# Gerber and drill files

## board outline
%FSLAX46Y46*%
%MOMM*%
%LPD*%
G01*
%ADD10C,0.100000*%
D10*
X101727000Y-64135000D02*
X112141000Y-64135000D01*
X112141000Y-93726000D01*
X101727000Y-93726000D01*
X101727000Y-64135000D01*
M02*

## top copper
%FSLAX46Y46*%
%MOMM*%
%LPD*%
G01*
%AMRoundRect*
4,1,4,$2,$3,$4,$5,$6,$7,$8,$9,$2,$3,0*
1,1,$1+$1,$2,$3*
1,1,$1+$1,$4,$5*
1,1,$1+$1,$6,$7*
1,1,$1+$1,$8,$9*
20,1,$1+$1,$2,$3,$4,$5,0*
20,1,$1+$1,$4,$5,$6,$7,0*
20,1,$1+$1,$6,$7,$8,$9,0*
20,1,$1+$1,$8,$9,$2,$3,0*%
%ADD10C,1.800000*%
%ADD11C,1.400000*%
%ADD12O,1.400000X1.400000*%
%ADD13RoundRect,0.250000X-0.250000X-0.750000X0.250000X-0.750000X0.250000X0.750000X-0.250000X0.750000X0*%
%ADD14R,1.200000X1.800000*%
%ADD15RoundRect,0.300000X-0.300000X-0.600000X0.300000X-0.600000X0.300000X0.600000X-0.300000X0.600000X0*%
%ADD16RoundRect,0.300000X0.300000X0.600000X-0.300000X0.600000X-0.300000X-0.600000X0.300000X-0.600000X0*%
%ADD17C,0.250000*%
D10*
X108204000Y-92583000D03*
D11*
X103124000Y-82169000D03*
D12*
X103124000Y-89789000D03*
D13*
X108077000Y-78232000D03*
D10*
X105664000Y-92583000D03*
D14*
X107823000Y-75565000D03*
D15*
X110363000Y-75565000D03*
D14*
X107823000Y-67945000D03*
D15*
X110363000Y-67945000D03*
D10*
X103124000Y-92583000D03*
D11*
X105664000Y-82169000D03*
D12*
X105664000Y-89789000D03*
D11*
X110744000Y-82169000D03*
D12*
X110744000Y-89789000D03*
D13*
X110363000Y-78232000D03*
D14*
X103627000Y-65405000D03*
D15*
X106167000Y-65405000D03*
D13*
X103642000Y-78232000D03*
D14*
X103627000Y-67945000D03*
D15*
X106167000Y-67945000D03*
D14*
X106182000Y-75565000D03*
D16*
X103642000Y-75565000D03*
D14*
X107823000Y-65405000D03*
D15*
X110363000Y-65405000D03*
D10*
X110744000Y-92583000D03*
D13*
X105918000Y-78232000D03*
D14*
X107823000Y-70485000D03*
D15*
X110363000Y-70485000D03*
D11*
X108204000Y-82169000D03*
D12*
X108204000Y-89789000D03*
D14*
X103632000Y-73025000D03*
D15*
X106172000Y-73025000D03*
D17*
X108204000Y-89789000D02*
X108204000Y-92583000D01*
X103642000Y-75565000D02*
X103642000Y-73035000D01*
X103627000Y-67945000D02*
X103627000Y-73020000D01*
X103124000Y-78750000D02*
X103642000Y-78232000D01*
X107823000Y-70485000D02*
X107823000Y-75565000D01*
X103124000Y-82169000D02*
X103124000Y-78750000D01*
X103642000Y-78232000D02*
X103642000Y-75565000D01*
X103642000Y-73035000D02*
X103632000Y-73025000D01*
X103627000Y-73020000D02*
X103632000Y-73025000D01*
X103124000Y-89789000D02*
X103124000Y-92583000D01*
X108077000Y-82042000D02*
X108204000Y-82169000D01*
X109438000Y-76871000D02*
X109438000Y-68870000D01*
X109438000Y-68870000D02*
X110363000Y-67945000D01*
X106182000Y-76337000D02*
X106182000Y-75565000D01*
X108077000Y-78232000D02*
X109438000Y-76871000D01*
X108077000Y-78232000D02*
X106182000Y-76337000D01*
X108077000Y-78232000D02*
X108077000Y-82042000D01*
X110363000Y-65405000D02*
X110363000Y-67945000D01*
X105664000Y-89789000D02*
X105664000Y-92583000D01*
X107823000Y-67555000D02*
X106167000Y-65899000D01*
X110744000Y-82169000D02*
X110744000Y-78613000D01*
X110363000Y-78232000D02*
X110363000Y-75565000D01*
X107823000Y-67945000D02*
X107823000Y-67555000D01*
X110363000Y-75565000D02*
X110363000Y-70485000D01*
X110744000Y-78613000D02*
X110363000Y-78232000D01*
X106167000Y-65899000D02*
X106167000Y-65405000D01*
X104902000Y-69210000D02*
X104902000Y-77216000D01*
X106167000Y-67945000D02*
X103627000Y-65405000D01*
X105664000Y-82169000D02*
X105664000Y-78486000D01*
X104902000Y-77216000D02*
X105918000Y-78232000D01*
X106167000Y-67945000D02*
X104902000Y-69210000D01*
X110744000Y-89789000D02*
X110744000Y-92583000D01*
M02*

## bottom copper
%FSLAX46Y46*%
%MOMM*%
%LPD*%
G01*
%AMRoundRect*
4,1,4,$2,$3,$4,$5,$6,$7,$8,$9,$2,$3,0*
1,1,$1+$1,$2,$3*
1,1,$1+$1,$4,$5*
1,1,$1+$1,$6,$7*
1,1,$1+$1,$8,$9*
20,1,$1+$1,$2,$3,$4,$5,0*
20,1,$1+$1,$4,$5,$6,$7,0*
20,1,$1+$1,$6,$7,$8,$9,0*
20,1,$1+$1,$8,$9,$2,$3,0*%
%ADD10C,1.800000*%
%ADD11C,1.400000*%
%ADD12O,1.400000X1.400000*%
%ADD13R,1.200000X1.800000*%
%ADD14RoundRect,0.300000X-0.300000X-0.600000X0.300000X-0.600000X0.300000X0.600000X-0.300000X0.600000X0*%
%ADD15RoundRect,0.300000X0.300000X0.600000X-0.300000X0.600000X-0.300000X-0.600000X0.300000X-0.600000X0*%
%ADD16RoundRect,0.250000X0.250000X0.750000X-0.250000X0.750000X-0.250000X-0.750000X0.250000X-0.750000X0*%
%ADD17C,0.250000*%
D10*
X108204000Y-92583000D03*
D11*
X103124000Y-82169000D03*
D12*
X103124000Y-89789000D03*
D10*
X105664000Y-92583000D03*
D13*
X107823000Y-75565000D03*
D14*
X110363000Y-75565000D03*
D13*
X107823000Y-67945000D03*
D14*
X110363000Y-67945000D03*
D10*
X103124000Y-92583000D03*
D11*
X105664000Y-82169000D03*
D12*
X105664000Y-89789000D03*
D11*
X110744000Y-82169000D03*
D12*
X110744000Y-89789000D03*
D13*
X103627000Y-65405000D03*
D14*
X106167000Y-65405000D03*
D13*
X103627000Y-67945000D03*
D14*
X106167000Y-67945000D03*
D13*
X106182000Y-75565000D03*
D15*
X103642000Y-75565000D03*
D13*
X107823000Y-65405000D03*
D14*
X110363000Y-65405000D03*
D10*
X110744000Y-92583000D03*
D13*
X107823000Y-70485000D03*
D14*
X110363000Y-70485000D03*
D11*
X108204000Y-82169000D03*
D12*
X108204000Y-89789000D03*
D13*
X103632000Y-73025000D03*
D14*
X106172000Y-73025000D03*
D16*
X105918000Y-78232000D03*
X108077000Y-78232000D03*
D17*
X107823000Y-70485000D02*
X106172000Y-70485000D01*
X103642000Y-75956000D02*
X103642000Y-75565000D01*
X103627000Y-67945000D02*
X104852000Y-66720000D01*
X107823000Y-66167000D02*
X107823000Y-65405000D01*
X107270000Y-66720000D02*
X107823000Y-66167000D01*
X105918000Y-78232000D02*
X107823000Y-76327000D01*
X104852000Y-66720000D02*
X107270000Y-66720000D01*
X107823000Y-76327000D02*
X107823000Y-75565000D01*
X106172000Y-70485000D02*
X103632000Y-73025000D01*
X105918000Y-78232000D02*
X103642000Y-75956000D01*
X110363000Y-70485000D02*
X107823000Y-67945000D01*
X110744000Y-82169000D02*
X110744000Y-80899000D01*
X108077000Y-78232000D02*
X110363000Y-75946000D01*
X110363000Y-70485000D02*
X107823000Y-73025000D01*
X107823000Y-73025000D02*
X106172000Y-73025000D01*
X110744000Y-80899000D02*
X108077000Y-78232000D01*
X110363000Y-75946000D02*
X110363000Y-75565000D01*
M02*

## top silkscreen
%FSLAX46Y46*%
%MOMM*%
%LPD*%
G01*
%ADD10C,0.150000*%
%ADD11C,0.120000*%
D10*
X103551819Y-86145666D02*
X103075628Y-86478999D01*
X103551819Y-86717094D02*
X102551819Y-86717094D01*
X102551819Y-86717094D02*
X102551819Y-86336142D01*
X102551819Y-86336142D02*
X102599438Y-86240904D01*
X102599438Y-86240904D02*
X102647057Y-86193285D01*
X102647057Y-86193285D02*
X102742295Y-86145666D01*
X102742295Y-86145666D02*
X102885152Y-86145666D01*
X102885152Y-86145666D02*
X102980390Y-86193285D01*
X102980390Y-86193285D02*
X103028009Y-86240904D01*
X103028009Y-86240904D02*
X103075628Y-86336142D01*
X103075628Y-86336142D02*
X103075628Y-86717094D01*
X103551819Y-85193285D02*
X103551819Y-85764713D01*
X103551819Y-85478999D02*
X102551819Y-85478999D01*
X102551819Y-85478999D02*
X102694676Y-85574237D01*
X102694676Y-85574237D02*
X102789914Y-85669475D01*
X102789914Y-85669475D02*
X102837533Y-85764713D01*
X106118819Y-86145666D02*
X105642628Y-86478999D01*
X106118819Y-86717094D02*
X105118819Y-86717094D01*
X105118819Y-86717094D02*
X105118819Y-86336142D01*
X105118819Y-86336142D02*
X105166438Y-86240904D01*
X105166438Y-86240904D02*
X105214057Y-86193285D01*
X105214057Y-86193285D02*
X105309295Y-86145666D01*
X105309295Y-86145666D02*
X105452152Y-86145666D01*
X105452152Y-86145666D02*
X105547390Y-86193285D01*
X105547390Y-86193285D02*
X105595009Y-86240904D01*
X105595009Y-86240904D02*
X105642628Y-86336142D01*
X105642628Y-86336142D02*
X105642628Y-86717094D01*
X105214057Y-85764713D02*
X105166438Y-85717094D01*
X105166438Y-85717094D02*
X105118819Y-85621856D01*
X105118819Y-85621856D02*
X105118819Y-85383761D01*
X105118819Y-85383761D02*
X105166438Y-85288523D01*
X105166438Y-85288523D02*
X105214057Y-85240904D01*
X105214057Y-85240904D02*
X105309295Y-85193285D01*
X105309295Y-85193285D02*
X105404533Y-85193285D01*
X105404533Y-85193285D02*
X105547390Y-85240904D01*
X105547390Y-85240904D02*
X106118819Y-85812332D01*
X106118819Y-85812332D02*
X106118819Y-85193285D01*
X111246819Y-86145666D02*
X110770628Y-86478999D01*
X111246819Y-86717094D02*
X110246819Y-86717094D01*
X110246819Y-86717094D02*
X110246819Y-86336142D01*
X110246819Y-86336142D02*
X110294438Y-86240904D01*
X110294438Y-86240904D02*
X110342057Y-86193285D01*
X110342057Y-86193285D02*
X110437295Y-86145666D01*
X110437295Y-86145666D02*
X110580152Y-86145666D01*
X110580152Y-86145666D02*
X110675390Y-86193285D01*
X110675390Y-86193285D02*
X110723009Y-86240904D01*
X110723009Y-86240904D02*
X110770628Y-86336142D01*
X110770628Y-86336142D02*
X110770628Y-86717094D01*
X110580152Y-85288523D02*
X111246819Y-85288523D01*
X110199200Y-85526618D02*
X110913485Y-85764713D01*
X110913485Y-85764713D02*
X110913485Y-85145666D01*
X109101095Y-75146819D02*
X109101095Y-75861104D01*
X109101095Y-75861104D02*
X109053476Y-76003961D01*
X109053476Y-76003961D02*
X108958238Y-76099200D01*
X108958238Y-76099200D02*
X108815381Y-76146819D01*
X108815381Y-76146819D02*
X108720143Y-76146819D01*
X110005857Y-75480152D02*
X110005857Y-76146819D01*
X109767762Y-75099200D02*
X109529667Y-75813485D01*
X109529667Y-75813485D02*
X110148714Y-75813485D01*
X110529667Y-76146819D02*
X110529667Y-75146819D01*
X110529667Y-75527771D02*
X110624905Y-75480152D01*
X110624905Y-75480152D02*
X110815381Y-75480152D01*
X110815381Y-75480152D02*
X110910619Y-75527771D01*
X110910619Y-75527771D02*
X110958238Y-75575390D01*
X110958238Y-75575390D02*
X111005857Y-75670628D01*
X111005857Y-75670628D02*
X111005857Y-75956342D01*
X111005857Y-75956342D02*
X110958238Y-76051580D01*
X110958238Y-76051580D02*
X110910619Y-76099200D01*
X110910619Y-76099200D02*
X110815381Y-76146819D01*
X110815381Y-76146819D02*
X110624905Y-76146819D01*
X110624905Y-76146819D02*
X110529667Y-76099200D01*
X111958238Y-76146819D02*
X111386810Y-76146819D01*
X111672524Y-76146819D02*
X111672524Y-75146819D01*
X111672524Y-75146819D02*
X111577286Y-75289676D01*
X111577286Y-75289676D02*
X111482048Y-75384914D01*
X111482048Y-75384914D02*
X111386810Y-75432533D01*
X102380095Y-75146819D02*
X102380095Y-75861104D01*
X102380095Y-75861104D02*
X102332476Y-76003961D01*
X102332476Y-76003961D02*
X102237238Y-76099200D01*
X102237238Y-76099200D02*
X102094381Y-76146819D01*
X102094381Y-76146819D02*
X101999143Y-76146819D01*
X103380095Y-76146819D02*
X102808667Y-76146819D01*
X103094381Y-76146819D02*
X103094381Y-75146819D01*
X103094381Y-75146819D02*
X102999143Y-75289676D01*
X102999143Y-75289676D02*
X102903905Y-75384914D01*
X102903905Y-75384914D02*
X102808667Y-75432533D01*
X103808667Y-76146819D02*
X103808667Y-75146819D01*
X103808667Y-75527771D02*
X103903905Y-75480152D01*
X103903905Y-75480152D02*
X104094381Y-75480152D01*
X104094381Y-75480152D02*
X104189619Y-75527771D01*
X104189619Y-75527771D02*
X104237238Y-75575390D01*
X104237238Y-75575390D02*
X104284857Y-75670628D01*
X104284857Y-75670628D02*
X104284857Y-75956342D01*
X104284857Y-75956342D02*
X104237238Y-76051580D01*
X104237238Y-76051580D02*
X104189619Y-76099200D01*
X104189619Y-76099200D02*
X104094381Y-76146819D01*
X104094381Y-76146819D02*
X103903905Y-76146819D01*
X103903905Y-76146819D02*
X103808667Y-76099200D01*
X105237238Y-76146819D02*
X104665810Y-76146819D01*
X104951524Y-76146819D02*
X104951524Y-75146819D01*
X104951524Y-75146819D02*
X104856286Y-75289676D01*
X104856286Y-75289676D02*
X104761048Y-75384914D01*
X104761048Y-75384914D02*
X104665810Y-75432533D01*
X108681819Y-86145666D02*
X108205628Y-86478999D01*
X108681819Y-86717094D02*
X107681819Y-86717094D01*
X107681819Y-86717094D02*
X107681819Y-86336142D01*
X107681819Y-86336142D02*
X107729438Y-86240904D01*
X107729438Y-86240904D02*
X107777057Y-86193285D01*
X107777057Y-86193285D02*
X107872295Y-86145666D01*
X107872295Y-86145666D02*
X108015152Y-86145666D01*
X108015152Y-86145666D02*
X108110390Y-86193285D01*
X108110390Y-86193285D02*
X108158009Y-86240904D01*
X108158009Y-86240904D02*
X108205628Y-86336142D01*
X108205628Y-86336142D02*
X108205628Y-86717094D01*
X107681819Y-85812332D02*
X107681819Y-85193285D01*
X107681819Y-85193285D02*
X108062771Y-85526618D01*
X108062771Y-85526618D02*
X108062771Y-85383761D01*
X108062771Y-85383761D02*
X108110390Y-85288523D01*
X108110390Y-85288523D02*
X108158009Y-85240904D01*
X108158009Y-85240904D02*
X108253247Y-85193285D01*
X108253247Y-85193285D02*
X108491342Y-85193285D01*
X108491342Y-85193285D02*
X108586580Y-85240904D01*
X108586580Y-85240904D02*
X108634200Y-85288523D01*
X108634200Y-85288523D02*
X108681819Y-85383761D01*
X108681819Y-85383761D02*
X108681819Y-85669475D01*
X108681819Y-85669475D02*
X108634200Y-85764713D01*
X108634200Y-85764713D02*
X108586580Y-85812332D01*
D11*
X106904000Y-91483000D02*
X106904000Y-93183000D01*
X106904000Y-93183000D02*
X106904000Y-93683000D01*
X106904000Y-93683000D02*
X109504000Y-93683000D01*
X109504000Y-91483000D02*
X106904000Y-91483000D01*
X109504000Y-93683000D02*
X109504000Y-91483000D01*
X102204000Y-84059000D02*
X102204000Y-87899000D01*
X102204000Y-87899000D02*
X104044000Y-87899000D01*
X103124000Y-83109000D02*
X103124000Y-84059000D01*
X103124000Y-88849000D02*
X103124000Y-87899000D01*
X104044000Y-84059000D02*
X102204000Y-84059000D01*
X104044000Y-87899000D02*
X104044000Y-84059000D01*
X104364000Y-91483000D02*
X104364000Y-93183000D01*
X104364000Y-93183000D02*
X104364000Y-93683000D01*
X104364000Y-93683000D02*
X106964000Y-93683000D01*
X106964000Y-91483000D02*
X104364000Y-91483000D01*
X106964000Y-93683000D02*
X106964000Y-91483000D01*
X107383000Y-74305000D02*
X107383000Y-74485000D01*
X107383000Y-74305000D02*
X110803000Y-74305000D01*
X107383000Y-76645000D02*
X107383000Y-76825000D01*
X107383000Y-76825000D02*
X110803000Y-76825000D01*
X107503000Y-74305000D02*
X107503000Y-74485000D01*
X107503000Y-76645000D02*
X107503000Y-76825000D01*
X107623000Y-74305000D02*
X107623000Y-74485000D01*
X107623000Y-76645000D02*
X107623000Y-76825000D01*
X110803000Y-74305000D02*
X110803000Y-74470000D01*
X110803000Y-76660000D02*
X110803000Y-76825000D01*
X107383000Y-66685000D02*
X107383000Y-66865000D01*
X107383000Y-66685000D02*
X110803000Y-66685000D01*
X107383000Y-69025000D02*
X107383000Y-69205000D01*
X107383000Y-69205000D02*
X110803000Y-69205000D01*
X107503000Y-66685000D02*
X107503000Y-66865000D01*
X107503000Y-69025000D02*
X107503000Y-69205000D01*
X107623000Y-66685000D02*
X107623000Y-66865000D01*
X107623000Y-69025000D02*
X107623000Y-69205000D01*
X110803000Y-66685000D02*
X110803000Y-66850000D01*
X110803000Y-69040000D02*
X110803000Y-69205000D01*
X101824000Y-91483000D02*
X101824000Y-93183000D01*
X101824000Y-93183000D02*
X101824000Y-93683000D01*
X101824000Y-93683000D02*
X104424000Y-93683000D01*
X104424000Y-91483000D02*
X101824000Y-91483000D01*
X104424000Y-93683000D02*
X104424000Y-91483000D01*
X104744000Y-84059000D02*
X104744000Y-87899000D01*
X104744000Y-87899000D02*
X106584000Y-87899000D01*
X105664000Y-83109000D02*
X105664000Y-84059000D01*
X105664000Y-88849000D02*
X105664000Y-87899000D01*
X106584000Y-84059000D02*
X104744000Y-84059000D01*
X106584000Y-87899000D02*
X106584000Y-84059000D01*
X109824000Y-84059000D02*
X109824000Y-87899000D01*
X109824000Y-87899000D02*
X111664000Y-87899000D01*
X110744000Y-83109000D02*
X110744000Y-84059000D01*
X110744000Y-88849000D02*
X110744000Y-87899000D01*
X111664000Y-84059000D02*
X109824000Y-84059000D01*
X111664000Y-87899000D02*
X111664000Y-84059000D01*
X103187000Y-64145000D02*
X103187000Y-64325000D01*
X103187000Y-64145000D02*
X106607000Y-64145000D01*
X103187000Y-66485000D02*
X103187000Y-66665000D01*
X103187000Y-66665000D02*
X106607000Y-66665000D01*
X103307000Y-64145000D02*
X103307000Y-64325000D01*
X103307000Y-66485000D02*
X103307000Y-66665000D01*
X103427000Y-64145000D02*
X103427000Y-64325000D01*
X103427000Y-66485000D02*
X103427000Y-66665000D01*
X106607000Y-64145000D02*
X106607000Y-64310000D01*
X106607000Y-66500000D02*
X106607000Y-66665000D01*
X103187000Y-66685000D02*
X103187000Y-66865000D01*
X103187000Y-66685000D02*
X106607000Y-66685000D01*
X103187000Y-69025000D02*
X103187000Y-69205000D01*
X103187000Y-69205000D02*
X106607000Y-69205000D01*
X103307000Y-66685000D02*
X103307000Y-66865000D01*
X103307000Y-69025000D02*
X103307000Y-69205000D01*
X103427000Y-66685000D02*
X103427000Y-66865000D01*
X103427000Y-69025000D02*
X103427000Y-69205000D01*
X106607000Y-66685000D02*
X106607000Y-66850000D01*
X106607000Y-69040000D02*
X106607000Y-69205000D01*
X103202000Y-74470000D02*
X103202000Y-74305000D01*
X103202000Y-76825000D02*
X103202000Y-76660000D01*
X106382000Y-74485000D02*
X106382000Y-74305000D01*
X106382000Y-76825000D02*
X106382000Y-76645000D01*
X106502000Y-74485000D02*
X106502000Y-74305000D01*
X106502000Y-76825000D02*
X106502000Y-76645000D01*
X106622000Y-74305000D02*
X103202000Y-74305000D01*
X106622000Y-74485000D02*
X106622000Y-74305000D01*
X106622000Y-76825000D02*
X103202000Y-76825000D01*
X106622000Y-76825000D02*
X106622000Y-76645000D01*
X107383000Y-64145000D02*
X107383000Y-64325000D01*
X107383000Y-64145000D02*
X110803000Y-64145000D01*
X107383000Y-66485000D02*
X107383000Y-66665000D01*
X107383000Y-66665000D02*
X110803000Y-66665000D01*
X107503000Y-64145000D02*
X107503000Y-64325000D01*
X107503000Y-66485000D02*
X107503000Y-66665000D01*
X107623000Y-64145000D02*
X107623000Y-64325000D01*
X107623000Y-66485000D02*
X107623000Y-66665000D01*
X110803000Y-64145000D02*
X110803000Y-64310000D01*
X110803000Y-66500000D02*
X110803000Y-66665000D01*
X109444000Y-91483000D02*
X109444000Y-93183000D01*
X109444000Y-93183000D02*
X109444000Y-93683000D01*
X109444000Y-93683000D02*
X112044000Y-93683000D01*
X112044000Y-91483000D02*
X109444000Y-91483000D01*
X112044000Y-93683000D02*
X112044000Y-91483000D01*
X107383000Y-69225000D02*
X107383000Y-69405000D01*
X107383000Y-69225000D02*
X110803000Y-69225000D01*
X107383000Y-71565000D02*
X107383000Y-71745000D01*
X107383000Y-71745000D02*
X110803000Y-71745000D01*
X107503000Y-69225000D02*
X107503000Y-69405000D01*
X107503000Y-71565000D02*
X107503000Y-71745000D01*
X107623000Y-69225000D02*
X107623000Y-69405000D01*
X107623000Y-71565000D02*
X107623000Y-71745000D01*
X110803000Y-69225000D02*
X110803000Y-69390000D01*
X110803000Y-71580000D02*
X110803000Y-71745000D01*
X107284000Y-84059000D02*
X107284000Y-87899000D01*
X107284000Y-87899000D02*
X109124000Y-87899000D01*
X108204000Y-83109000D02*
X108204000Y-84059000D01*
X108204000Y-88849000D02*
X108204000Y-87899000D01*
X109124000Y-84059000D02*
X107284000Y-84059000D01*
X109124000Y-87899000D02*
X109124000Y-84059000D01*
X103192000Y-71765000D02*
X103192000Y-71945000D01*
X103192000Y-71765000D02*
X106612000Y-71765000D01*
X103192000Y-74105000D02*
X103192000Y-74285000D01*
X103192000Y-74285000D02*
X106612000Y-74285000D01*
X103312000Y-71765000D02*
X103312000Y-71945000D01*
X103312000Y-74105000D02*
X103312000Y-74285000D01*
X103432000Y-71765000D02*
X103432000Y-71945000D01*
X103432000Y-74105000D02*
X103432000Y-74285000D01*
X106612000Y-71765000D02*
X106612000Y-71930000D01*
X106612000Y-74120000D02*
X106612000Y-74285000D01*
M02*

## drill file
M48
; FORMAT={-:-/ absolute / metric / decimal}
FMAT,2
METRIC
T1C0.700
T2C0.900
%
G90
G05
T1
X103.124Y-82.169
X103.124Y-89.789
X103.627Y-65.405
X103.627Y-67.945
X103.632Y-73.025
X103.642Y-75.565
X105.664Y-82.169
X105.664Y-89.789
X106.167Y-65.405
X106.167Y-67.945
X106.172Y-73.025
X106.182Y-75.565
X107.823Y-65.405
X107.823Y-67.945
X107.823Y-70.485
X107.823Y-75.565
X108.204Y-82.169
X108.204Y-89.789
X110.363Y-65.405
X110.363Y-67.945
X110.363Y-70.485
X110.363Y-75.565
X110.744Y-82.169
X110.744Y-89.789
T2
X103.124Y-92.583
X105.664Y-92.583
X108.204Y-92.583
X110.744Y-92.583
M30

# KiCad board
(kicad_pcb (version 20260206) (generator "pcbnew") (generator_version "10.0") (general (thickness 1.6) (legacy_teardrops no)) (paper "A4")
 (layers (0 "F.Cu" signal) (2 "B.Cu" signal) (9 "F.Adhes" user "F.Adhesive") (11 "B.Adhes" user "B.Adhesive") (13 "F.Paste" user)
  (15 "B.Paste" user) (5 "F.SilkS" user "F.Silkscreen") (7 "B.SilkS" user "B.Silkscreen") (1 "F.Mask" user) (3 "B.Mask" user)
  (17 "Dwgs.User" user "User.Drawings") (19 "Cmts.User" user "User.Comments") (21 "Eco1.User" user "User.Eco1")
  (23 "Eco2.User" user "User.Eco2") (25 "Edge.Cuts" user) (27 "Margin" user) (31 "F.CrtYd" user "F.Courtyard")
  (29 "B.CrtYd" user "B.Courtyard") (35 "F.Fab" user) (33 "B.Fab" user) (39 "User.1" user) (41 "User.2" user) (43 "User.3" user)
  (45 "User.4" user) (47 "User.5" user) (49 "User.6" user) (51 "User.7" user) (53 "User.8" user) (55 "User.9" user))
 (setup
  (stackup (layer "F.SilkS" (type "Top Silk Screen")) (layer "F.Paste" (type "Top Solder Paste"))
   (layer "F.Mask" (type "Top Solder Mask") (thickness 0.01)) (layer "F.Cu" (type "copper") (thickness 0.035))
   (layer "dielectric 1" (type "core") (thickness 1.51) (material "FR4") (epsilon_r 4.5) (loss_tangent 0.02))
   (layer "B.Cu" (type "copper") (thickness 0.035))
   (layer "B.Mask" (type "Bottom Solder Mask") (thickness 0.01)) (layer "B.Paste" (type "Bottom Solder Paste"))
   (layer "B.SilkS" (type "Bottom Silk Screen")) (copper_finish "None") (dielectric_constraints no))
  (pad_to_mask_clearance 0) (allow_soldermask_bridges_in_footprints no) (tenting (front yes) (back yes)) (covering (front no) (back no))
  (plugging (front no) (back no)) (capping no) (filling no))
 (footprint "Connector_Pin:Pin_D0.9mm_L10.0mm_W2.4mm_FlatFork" (layer "F.Cu") (at 108.204 92.583)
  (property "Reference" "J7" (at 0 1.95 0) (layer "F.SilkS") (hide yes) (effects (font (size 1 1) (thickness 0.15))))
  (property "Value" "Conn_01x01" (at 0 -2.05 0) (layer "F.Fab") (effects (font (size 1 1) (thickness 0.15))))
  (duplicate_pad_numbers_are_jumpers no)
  (fp_line (start -1.3 -1.1) (end -1.3 0.6) (stroke (width 0.12) (type solid)) (layer "F.SilkS"))
  (fp_line (start -1.3 0.6) (end -1.3 1.1) (stroke (width 0.12) (type solid)) (layer "F.SilkS"))
  (fp_line (start -1.3 1.1) (end 1.3 1.1) (stroke (width 0.12) (type solid)) (layer "F.SilkS"))
  (fp_line (start 1.3 -1.1) (end -1.3 -1.1) (stroke (width 0.12) (type solid)) (layer "F.SilkS"))
  (fp_line (start 1.3 1.1) (end 1.3 -1.1) (stroke (width 0.12) (type solid)) (layer "F.SilkS"))
  (pad "1" thru_hole circle (at 0 0) (size 1.8 1.8) (drill 0.9) (layers "*.Cu" "*.Mask") (remove_unused_layers no) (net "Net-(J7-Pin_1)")))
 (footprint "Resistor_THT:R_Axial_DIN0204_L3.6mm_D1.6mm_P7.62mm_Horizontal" (layer "F.Cu") (at 103.124 82.169 -90)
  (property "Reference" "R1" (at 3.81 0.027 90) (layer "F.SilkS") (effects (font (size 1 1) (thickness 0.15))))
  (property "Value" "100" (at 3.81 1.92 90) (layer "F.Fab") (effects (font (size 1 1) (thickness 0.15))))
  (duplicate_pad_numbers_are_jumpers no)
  (fp_line (start 1.89 0.92) (end 5.73 0.92) (stroke (width 0.12) (type solid)) (layer "F.SilkS"))
  (fp_line (start 5.73 0.92) (end 5.73 -0.92) (stroke (width 0.12) (type solid)) (layer "F.SilkS"))
  (fp_line (start 0.94 0) (end 1.89 0) (stroke (width 0.12) (type solid)) (layer "F.SilkS"))
  (fp_line (start 6.68 0) (end 5.73 0) (stroke (width 0.12) (type solid)) (layer "F.SilkS"))
  (fp_line (start 1.89 -0.92) (end 1.89 0.92) (stroke (width 0.12) (type solid)) (layer "F.SilkS"))
  (fp_line (start 5.73 -0.92) (end 1.89 -0.92) (stroke (width 0.12) (type solid)) (layer "F.SilkS"))
  (pad "1" thru_hole circle (at 0 0 270) (size 1.4 1.4) (drill 0.7) (layers "*.Cu" "*.Mask") (remove_unused_layers no) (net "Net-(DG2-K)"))
  (pad "2" thru_hole oval (at 7.62 0 270) (size 1.4 1.4) (drill 0.7) (layers "*.Cu" "*.Mask") (remove_unused_layers no)
   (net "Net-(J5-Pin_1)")))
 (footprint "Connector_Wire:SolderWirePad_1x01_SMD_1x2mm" (layer "F.Cu") (at 108.077 78.232)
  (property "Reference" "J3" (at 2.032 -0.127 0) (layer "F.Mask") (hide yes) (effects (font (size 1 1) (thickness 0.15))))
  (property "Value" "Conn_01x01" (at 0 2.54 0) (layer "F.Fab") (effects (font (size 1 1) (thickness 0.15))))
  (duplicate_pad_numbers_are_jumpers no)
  (pad "1" smd roundrect (at 0 0) (size 1 2) (layers "F.Cu" "F.Mask" "F.Paste") (roundrect_rratio 0.25) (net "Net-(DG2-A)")))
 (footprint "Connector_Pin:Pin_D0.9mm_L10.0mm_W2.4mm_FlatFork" (layer "F.Cu") (at 105.664 92.583)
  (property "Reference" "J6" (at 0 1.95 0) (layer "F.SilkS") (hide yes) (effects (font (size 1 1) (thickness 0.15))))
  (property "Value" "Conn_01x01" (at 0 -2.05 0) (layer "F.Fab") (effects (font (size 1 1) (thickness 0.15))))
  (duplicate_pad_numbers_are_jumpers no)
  (fp_line (start -1.3 -1.1) (end -1.3 0.6) (stroke (width 0.12) (type solid)) (layer "F.SilkS"))
  (fp_line (start -1.3 0.6) (end -1.3 1.1) (stroke (width 0.12) (type solid)) (layer "F.SilkS"))
  (fp_line (start -1.3 1.1) (end 1.3 1.1) (stroke (width 0.12) (type solid)) (layer "F.SilkS"))
  (fp_line (start 1.3 -1.1) (end -1.3 -1.1) (stroke (width 0.12) (type solid)) (layer "F.SilkS"))
  (fp_line (start 1.3 1.1) (end 1.3 -1.1) (stroke (width 0.12) (type solid)) (layer "F.SilkS"))
  (pad "1" thru_hole circle (at 0 0) (size 1.8 1.8) (drill 0.9) (layers "*.Cu" "*.Mask") (remove_unused_layers no) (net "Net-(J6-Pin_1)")))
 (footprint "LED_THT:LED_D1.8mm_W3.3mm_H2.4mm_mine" (layer "F.Cu") (at 107.823 75.565)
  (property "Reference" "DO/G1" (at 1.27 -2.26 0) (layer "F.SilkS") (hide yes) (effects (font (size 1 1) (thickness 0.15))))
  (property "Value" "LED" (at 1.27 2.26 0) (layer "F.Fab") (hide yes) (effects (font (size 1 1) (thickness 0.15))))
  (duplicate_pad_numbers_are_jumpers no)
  (fp_line (start -0.44 -1.26) (end -0.44 -1.08) (stroke (width 0.12) (type solid)) (layer "F.SilkS"))
  (fp_line (start -0.44 -1.26) (end 2.98 -1.26) (stroke (width 0.12) (type solid)) (layer "F.SilkS"))
  (fp_line (start -0.44 1.08) (end -0.44 1.26) (stroke (width 0.12) (type solid)) (layer "F.SilkS"))
  (fp_line (start -0.44 1.26) (end 2.98 1.26) (stroke (width 0.12) (type solid)) (layer "F.SilkS"))
  (fp_line (start -0.32 -1.26) (end -0.32 -1.08) (stroke (width 0.12) (type solid)) (layer "F.SilkS"))
  (fp_line (start -0.32 1.08) (end -0.32 1.26) (stroke (width 0.12) (type solid)) (layer "F.SilkS"))
  (fp_line (start -0.2 -1.26) (end -0.2 -1.08) (stroke (width 0.12) (type solid)) (layer "F.SilkS"))
  (fp_line (start -0.2 1.08) (end -0.2 1.26) (stroke (width 0.12) (type solid)) (layer "F.SilkS"))
  (fp_line (start 2.98 -1.26) (end 2.98 -1.095) (stroke (width 0.12) (type solid)) (layer "F.SilkS"))
  (fp_line (start 2.98 1.095) (end 2.98 1.26) (stroke (width 0.12) (type solid)) (layer "F.SilkS"))
  (pad "1" thru_hole rect (at 0 0) (size 1.2 1.8) (drill 0.7) (layers "*.Cu" "*.Mask") (remove_unused_layers no) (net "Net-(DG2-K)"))
  (pad "2" thru_hole roundrect (at 2.54 0) (size 1.2 1.8) (drill 0.7) (layers "*.Cu" "*.Mask") (remove_unused_layers no)
   (roundrect_rratio 0.25) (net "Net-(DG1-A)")))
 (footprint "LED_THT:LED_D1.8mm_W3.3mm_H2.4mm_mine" (layer "F.Cu") (at 107.823 67.945)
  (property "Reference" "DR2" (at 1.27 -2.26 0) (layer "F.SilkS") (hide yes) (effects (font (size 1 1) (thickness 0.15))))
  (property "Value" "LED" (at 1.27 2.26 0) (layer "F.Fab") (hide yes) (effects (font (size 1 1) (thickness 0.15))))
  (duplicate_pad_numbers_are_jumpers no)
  (fp_line (start -0.44 -1.26) (end -0.44 -1.08) (stroke (width 0.12) (type solid)) (layer "F.SilkS"))
  (fp_line (start -0.44 -1.26) (end 2.98 -1.26) (stroke (width 0.12) (type solid)) (layer "F.SilkS"))
  (fp_line (start -0.44 1.08) (end -0.44 1.26) (stroke (width 0.12) (type solid)) (layer "F.SilkS"))
  (fp_line (start -0.44 1.26) (end 2.98 1.26) (stroke (width 0.12) (type solid)) (layer "F.SilkS"))
  (fp_line (start -0.32 -1.26) (end -0.32 -1.08) (stroke (width 0.12) (type solid)) (layer "F.SilkS"))
  (fp_line (start -0.32 1.08) (end -0.32 1.26) (stroke (width 0.12) (type solid)) (layer "F.SilkS"))
  (fp_line (start -0.2 -1.26) (end -0.2 -1.08) (stroke (width 0.12) (type solid)) (layer "F.SilkS"))
  (fp_line (start -0.2 1.08) (end -0.2 1.26) (stroke (width 0.12) (type solid)) (layer "F.SilkS"))
  (fp_line (start 2.98 -1.26) (end 2.98 -1.095) (stroke (width 0.12) (type solid)) (layer "F.SilkS"))
  (fp_line (start 2.98 1.095) (end 2.98 1.26) (stroke (width 0.12) (type solid)) (layer "F.SilkS"))
  (pad "1" thru_hole rect (at 0 0) (size 1.2 1.8) (drill 0.7) (layers "*.Cu" "*.Mask") (remove_unused_layers no) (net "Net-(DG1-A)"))
  (pad "2" thru_hole roundrect (at 2.54 0) (size 1.2 1.8) (drill 0.7) (layers "*.Cu" "*.Mask") (remove_unused_layers no)
   (roundrect_rratio 0.25) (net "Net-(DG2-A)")))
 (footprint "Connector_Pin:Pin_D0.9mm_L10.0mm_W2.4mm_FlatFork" (layer "F.Cu") (at 103.124 92.583)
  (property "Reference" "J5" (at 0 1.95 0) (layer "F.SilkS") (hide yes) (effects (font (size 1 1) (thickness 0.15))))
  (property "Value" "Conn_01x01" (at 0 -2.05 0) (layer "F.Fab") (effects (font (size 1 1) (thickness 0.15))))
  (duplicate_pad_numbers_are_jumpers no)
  (fp_line (start -1.3 -1.1) (end -1.3 0.6) (stroke (width 0.12) (type solid)) (layer "F.SilkS"))
  (fp_line (start -1.3 0.6) (end -1.3 1.1) (stroke (width 0.12) (type solid)) (layer "F.SilkS"))
  (fp_line (start -1.3 1.1) (end 1.3 1.1) (stroke (width 0.12) (type solid)) (layer "F.SilkS"))
  (fp_line (start 1.3 -1.1) (end -1.3 -1.1) (stroke (width 0.12) (type solid)) (layer "F.SilkS"))
  (fp_line (start 1.3 1.1) (end 1.3 -1.1) (stroke (width 0.12) (type solid)) (layer "F.SilkS"))
  (pad "1" thru_hole circle (at 0 0) (size 1.8 1.8) (drill 0.9) (layers "*.Cu" "*.Mask") (remove_unused_layers no) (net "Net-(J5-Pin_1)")))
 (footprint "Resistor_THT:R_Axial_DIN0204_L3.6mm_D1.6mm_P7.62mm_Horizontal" (layer "F.Cu") (at 105.664 82.169 -90)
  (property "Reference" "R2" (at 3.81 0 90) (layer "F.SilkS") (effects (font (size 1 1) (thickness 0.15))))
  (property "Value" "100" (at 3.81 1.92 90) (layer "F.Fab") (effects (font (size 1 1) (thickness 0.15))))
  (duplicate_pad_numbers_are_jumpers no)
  (fp_line (start 1.89 0.92) (end 5.73 0.92) (stroke (width 0.12) (type solid)) (layer "F.SilkS"))
  (fp_line (start 5.73 0.92) (end 5.73 -0.92) (stroke (width 0.12) (type solid)) (layer "F.SilkS"))
  (fp_line (start 0.94 0) (end 1.89 0) (stroke (width 0.12) (type solid)) (layer "F.SilkS"))
  (fp_line (start 6.68 0) (end 5.73 0) (stroke (width 0.12) (type solid)) (layer "F.SilkS"))
  (fp_line (start 1.89 -0.92) (end 1.89 0.92) (stroke (width 0.12) (type solid)) (layer "F.SilkS"))
  (fp_line (start 5.73 -0.92) (end 1.89 -0.92) (stroke (width 0.12) (type solid)) (layer "F.SilkS"))
  (pad "1" thru_hole circle (at 0 0 270) (size 1.4 1.4) (drill 0.7) (layers "*.Cu" "*.Mask") (remove_unused_layers no) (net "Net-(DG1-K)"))
  (pad "2" thru_hole oval (at 7.62 0 270) (size 1.4 1.4) (drill 0.7) (layers "*.Cu" "*.Mask") (remove_unused_layers no)
   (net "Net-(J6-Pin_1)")))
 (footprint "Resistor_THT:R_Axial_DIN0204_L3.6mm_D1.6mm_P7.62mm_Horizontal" (layer "F.Cu") (at 110.744 82.169 -90)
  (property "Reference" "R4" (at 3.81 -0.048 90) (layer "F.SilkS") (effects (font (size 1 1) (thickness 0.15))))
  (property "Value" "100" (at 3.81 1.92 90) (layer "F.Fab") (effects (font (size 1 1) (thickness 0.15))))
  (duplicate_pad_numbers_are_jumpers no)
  (fp_line (start 1.89 0.92) (end 5.73 0.92) (stroke (width 0.12) (type solid)) (layer "F.SilkS"))
  (fp_line (start 5.73 0.92) (end 5.73 -0.92) (stroke (width 0.12) (type solid)) (layer "F.SilkS"))
  (fp_line (start 0.94 0) (end 1.89 0) (stroke (width 0.12) (type solid)) (layer "F.SilkS"))
  (fp_line (start 6.68 0) (end 5.73 0) (stroke (width 0.12) (type solid)) (layer "F.SilkS"))
  (fp_line (start 1.89 -0.92) (end 1.89 0.92) (stroke (width 0.12) (type solid)) (layer "F.SilkS"))
  (fp_line (start 5.73 -0.92) (end 1.89 -0.92) (stroke (width 0.12) (type solid)) (layer "F.SilkS"))
  (pad "1" thru_hole circle (at 0 0 270) (size 1.4 1.4) (drill 0.7) (layers "*.Cu" "*.Mask") (remove_unused_layers no) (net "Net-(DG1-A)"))
  (pad "2" thru_hole oval (at 7.62 0 270) (size 1.4 1.4) (drill 0.7) (layers "*.Cu" "*.Mask") (remove_unused_layers no)
   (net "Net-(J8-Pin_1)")))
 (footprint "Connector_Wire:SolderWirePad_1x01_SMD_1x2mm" (layer "F.Cu") (at 110.363 78.232)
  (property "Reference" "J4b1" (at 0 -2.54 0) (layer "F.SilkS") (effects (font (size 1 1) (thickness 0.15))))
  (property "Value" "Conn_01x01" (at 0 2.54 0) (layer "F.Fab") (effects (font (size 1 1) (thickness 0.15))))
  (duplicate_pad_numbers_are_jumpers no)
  (pad "1" smd roundrect (at 0 0) (size 1 2) (layers "F.Cu" "F.Mask" "F.Paste") (roundrect_rratio 0.25) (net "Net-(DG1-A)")))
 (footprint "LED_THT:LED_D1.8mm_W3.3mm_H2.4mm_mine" (layer "F.Cu") (at 103.627 65.405)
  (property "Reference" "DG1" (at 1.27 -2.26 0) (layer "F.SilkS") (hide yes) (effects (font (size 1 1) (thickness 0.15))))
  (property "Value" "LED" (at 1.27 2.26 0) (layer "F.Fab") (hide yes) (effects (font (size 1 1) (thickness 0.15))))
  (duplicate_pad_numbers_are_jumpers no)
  (fp_line (start -0.44 -1.26) (end -0.44 -1.08) (stroke (width 0.12) (type solid)) (layer "F.SilkS"))
  (fp_line (start -0.44 -1.26) (end 2.98 -1.26) (stroke (width 0.12) (type solid)) (layer "F.SilkS"))
  (fp_line (start -0.44 1.08) (end -0.44 1.26) (stroke (width 0.12) (type solid)) (layer "F.SilkS"))
  (fp_line (start -0.44 1.26) (end 2.98 1.26) (stroke (width 0.12) (type solid)) (layer "F.SilkS"))
  (fp_line (start -0.32 -1.26) (end -0.32 -1.08) (stroke (width 0.12) (type solid)) (layer "F.SilkS"))
  (fp_line (start -0.32 1.08) (end -0.32 1.26) (stroke (width 0.12) (type solid)) (layer "F.SilkS"))
  (fp_line (start -0.2 -1.26) (end -0.2 -1.08) (stroke (width 0.12) (type solid)) (layer "F.SilkS"))
  (fp_line (start -0.2 1.08) (end -0.2 1.26) (stroke (width 0.12) (type solid)) (layer "F.SilkS"))
  (fp_line (start 2.98 -1.26) (end 2.98 -1.095) (stroke (width 0.12) (type solid)) (layer "F.SilkS"))
  (fp_line (start 2.98 1.095) (end 2.98 1.26) (stroke (width 0.12) (type solid)) (layer "F.SilkS"))
  (pad "1" thru_hole rect (at 0 0) (size 1.2 1.8) (drill 0.7) (layers "*.Cu" "*.Mask") (remove_unused_layers no) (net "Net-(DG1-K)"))
  (pad "2" thru_hole roundrect (at 2.54 0) (size 1.2 1.8) (drill 0.7) (layers "*.Cu" "*.Mask") (remove_unused_layers no)
   (roundrect_rratio 0.25) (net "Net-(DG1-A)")))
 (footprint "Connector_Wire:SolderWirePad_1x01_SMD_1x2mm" (layer "F.Cu") (at 103.642 78.232)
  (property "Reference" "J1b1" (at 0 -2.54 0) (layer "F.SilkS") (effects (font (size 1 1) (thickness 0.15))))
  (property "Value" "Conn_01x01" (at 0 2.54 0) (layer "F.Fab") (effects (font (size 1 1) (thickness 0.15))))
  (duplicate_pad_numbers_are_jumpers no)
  (pad "1" smd roundrect (at 0 0) (size 1 2) (layers "F.Cu" "F.Mask" "F.Paste") (roundrect_rratio 0.25) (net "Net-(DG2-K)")))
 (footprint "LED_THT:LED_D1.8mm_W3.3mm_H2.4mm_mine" (layer "F.Cu") (at 103.627 67.945)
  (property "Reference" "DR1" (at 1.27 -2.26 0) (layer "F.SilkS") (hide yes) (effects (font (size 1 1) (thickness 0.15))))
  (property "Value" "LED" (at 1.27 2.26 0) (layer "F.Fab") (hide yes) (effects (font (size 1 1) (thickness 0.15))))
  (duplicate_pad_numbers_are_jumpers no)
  (fp_line (start -0.44 -1.26) (end -0.44 -1.08) (stroke (width 0.12) (type solid)) (layer "F.SilkS"))
  (fp_line (start -0.44 -1.26) (end 2.98 -1.26) (stroke (width 0.12) (type solid)) (layer "F.SilkS"))
  (fp_line (start -0.44 1.08) (end -0.44 1.26) (stroke (width 0.12) (type solid)) (layer "F.SilkS"))
  (fp_line (start -0.44 1.26) (end 2.98 1.26) (stroke (width 0.12) (type solid)) (layer "F.SilkS"))
  (fp_line (start -0.32 -1.26) (end -0.32 -1.08) (stroke (width 0.12) (type solid)) (layer "F.SilkS"))
  (fp_line (start -0.32 1.08) (end -0.32 1.26) (stroke (width 0.12) (type solid)) (layer "F.SilkS"))
  (fp_line (start -0.2 -1.26) (end -0.2 -1.08) (stroke (width 0.12) (type solid)) (layer "F.SilkS"))
  (fp_line (start -0.2 1.08) (end -0.2 1.26) (stroke (width 0.12) (type solid)) (layer "F.SilkS"))
  (fp_line (start 2.98 -1.26) (end 2.98 -1.095) (stroke (width 0.12) (type solid)) (layer "F.SilkS"))
  (fp_line (start 2.98 1.095) (end 2.98 1.26) (stroke (width 0.12) (type solid)) (layer "F.SilkS"))
  (pad "1" thru_hole rect (at 0 0) (size 1.2 1.8) (drill 0.7) (layers "*.Cu" "*.Mask") (remove_unused_layers no) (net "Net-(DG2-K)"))
  (pad "2" thru_hole roundrect (at 2.54 0) (size 1.2 1.8) (drill 0.7) (layers "*.Cu" "*.Mask") (remove_unused_layers no)
   (roundrect_rratio 0.25) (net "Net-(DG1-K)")))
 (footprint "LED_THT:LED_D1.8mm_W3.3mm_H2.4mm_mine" (layer "F.Cu") (at 106.182 75.565 180)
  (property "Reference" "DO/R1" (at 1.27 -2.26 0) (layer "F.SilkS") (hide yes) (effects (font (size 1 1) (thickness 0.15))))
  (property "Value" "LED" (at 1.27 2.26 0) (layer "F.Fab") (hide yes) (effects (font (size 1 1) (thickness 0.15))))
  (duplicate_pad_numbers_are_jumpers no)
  (fp_line (start 2.98 1.095) (end 2.98 1.26) (stroke (width 0.12) (type solid)) (layer "F.SilkS"))
  (fp_line (start 2.98 -1.26) (end 2.98 -1.095) (stroke (width 0.12) (type solid)) (layer "F.SilkS"))
  (fp_line (start -0.2 1.08) (end -0.2 1.26) (stroke (width 0.12) (type solid)) (layer "F.SilkS"))
  (fp_line (start -0.2 -1.26) (end -0.2 -1.08) (stroke (width 0.12) (type solid)) (layer "F.SilkS"))
  (fp_line (start -0.32 1.08) (end -0.32 1.26) (stroke (width 0.12) (type solid)) (layer "F.SilkS"))
  (fp_line (start -0.32 -1.26) (end -0.32 -1.08) (stroke (width 0.12) (type solid)) (layer "F.SilkS"))
  (fp_line (start -0.44 1.26) (end 2.98 1.26) (stroke (width 0.12) (type solid)) (layer "F.SilkS"))
  (fp_line (start -0.44 1.08) (end -0.44 1.26) (stroke (width 0.12) (type solid)) (layer "F.SilkS"))
  (fp_line (start -0.44 -1.26) (end 2.98 -1.26) (stroke (width 0.12) (type solid)) (layer "F.SilkS"))
  (fp_line (start -0.44 -1.26) (end -0.44 -1.08) (stroke (width 0.12) (type solid)) (layer "F.SilkS"))
  (pad "1" thru_hole rect (at 0 0 180) (size 1.2 1.8) (drill 0.7) (layers "*.Cu" "*.Mask") (remove_unused_layers no) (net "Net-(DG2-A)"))
  (pad "2" thru_hole roundrect (at 2.54 0 180) (size 1.2 1.8) (drill 0.7) (layers "*.Cu" "*.Mask") (remove_unused_layers no)
   (roundrect_rratio 0.25) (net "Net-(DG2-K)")))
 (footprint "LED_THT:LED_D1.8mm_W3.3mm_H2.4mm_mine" (layer "F.Cu") (at 107.823 65.405)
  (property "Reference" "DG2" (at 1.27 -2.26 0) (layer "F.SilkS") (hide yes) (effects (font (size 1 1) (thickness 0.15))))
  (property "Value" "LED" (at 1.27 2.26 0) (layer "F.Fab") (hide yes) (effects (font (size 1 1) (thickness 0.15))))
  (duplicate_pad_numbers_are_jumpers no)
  (fp_line (start -0.44 -1.26) (end -0.44 -1.08) (stroke (width 0.12) (type solid)) (layer "F.SilkS"))
  (fp_line (start -0.44 -1.26) (end 2.98 -1.26) (stroke (width 0.12) (type solid)) (layer "F.SilkS"))
  (fp_line (start -0.44 1.08) (end -0.44 1.26) (stroke (width 0.12) (type solid)) (layer "F.SilkS"))
  (fp_line (start -0.44 1.26) (end 2.98 1.26) (stroke (width 0.12) (type solid)) (layer "F.SilkS"))
  (fp_line (start -0.32 -1.26) (end -0.32 -1.08) (stroke (width 0.12) (type solid)) (layer "F.SilkS"))
  (fp_line (start -0.32 1.08) (end -0.32 1.26) (stroke (width 0.12) (type solid)) (layer "F.SilkS"))
  (fp_line (start -0.2 -1.26) (end -0.2 -1.08) (stroke (width 0.12) (type solid)) (layer "F.SilkS"))
  (fp_line (start -0.2 1.08) (end -0.2 1.26) (stroke (width 0.12) (type solid)) (layer "F.SilkS"))
  (fp_line (start 2.98 -1.26) (end 2.98 -1.095) (stroke (width 0.12) (type solid)) (layer "F.SilkS"))
  (fp_line (start 2.98 1.095) (end 2.98 1.26) (stroke (width 0.12) (type solid)) (layer "F.SilkS"))
  (pad "1" thru_hole rect (at 0 0) (size 1.2 1.8) (drill 0.7) (layers "*.Cu" "*.Mask") (remove_unused_layers no) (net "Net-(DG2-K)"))
  (pad "2" thru_hole roundrect (at 2.54 0) (size 1.2 1.8) (drill 0.7) (layers "*.Cu" "*.Mask") (remove_unused_layers no)
   (roundrect_rratio 0.25) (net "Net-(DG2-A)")))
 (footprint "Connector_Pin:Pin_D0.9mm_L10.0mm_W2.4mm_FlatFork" (layer "F.Cu") (at 110.744 92.583)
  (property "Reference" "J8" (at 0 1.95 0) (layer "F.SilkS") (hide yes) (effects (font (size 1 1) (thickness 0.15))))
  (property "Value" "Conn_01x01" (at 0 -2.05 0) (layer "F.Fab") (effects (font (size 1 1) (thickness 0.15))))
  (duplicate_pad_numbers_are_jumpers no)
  (fp_line (start -1.3 -1.1) (end -1.3 0.6) (stroke (width 0.12) (type solid)) (layer "F.SilkS"))
  (fp_line (start -1.3 0.6) (end -1.3 1.1) (stroke (width 0.12) (type solid)) (layer "F.SilkS"))
  (fp_line (start -1.3 1.1) (end 1.3 1.1) (stroke (width 0.12) (type solid)) (layer "F.SilkS"))
  (fp_line (start 1.3 -1.1) (end -1.3 -1.1) (stroke (width 0.12) (type solid)) (layer "F.SilkS"))
  (fp_line (start 1.3 1.1) (end 1.3 -1.1) (stroke (width 0.12) (type solid)) (layer "F.SilkS"))
  (pad "1" thru_hole circle (at 0 0) (size 1.8 1.8) (drill 0.9) (layers "*.Cu" "*.Mask") (remove_unused_layers no) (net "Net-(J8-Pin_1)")))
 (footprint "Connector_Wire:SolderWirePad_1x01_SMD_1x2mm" (layer "F.Cu") (at 105.918 78.232)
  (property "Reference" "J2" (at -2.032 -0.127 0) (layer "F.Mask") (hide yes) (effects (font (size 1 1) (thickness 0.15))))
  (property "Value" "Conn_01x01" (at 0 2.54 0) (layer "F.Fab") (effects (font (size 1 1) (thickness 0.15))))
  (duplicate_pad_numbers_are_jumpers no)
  (pad "1" smd roundrect (at 0 0) (size 1 2) (layers "F.Cu" "F.Mask" "F.Paste") (roundrect_rratio 0.25) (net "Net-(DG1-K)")))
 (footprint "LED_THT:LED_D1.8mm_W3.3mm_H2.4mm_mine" (layer "F.Cu") (at 107.823 70.485)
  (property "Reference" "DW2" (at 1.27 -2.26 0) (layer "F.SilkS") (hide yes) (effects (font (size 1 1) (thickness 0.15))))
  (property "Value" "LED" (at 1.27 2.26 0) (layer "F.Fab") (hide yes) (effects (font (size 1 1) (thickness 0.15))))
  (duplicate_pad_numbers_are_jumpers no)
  (fp_line (start -0.44 -1.26) (end -0.44 -1.08) (stroke (width 0.12) (type solid)) (layer "F.SilkS"))
  (fp_line (start -0.44 -1.26) (end 2.98 -1.26) (stroke (width 0.12) (type solid)) (layer "F.SilkS"))
  (fp_line (start -0.44 1.08) (end -0.44 1.26) (stroke (width 0.12) (type solid)) (layer "F.SilkS"))
  (fp_line (start -0.44 1.26) (end 2.98 1.26) (stroke (width 0.12) (type solid)) (layer "F.SilkS"))
  (fp_line (start -0.32 -1.26) (end -0.32 -1.08) (stroke (width 0.12) (type solid)) (layer "F.SilkS"))
  (fp_line (start -0.32 1.08) (end -0.32 1.26) (stroke (width 0.12) (type solid)) (layer "F.SilkS"))
  (fp_line (start -0.2 -1.26) (end -0.2 -1.08) (stroke (width 0.12) (type solid)) (layer "F.SilkS"))
  (fp_line (start -0.2 1.08) (end -0.2 1.26) (stroke (width 0.12) (type solid)) (layer "F.SilkS"))
  (fp_line (start 2.98 -1.26) (end 2.98 -1.095) (stroke (width 0.12) (type solid)) (layer "F.SilkS"))
  (fp_line (start 2.98 1.095) (end 2.98 1.26) (stroke (width 0.12) (type solid)) (layer "F.SilkS"))
  (pad "1" thru_hole rect (at 0 0) (size 1.2 1.8) (drill 0.7) (layers "*.Cu" "*.Mask") (remove_unused_layers no) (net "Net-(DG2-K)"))
  (pad "2" thru_hole roundrect (at 2.54 0) (size 1.2 1.8) (drill 0.7) (layers "*.Cu" "*.Mask") (remove_unused_layers no)
   (roundrect_rratio 0.25) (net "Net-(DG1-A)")))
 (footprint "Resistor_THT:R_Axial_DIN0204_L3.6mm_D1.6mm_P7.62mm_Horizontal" (layer "F.Cu") (at 108.204 82.169 -90)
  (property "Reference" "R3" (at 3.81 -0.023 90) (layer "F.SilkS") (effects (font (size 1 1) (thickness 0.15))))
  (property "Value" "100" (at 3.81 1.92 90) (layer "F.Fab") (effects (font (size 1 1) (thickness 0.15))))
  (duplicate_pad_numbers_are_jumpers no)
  (fp_line (start 1.89 0.92) (end 5.73 0.92) (stroke (width 0.12) (type solid)) (layer "F.SilkS"))
  (fp_line (start 5.73 0.92) (end 5.73 -0.92) (stroke (width 0.12) (type solid)) (layer "F.SilkS"))
  (fp_line (start 0.94 0) (end 1.89 0) (stroke (width 0.12) (type solid)) (layer "F.SilkS"))
  (fp_line (start 6.68 0) (end 5.73 0) (stroke (width 0.12) (type solid)) (layer "F.SilkS"))
  (fp_line (start 1.89 -0.92) (end 1.89 0.92) (stroke (width 0.12) (type solid)) (layer "F.SilkS"))
  (fp_line (start 5.73 -0.92) (end 1.89 -0.92) (stroke (width 0.12) (type solid)) (layer "F.SilkS"))
  (pad "1" thru_hole circle (at 0 0 270) (size 1.4 1.4) (drill 0.7) (layers "*.Cu" "*.Mask") (remove_unused_layers no) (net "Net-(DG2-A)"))
  (pad "2" thru_hole oval (at 7.62 0 270) (size 1.4 1.4) (drill 0.7) (layers "*.Cu" "*.Mask") (remove_unused_layers no)
   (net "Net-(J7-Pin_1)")))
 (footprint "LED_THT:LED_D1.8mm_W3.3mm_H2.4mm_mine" (layer "F.Cu") (at 103.632 73.025)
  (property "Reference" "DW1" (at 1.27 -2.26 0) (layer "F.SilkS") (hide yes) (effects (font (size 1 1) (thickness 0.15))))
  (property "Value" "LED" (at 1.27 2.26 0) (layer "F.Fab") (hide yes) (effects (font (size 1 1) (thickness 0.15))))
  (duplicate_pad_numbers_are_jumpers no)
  (fp_line (start -0.44 -1.26) (end -0.44 -1.08) (stroke (width 0.12) (type solid)) (layer "F.SilkS"))
  (fp_line (start -0.44 -1.26) (end 2.98 -1.26) (stroke (width 0.12) (type solid)) (layer "F.SilkS"))
  (fp_line (start -0.44 1.08) (end -0.44 1.26) (stroke (width 0.12) (type solid)) (layer "F.SilkS"))
  (fp_line (start -0.44 1.26) (end 2.98 1.26) (stroke (width 0.12) (type solid)) (layer "F.SilkS"))
  (fp_line (start -0.32 -1.26) (end -0.32 -1.08) (stroke (width 0.12) (type solid)) (layer "F.SilkS"))
  (fp_line (start -0.32 1.08) (end -0.32 1.26) (stroke (width 0.12) (type solid)) (layer "F.SilkS"))
  (fp_line (start -0.2 -1.26) (end -0.2 -1.08) (stroke (width 0.12) (type solid)) (layer "F.SilkS"))
  (fp_line (start -0.2 1.08) (end -0.2 1.26) (stroke (width 0.12) (type solid)) (layer "F.SilkS"))
  (fp_line (start 2.98 -1.26) (end 2.98 -1.095) (stroke (width 0.12) (type solid)) (layer "F.SilkS"))
  (fp_line (start 2.98 1.095) (end 2.98 1.26) (stroke (width 0.12) (type solid)) (layer "F.SilkS"))
  (pad "1" thru_hole rect (at 0 0) (size 1.2 1.8) (drill 0.7) (layers "*.Cu" "*.Mask") (remove_unused_layers no) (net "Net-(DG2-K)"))
  (pad "2" thru_hole roundrect (at 2.54 0) (size 1.2 1.8) (drill 0.7) (layers "*.Cu" "*.Mask") (remove_unused_layers no)
   (roundrect_rratio 0.25) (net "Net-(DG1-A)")))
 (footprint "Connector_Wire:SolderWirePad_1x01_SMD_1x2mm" (layer "B.Cu") (at 105.918 78.232 180)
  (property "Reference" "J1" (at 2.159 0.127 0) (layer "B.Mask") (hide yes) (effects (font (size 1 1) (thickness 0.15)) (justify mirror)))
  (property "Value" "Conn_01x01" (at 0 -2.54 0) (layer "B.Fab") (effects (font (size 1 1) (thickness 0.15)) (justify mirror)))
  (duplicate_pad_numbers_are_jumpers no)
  (pad "1" smd roundrect (at 0 0 180) (size 1 2) (layers "B.Cu" "B.Mask" "B.Paste") (roundrect_rratio 0.25) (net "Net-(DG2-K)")))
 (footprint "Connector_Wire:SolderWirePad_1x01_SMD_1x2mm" (layer "B.Cu") (at 108.077 78.232 180)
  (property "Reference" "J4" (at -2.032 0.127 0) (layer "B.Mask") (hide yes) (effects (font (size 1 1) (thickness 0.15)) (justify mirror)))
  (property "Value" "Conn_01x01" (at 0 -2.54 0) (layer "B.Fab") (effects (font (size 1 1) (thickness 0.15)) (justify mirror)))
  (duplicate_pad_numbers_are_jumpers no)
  (pad "1" smd roundrect (at 0 0 180) (size 1 2) (layers "B.Cu" "B.Mask" "B.Paste") (roundrect_rratio 0.25) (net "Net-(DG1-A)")))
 (gr_rect (start 101.727 64.135) (end 112.141 93.726) (stroke (width 0.1) (type default)) (fill no) (layer "Edge.Cuts"))
 (segment (start 108.204 89.789) (end 108.204 92.583) (width 0.25) (layer "F.Cu") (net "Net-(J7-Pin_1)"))
 (segment (start 103.642 75.565) (end 103.642 73.035) (width 0.25) (layer "F.Cu") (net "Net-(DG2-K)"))
 (segment (start 103.627 67.945) (end 103.627 73.02) (width 0.25) (layer "F.Cu") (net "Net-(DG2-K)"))
 (segment (start 103.124 78.75) (end 103.642 78.232) (width 0.25) (layer "F.Cu") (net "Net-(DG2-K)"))
 (segment (start 107.823 70.485) (end 107.823 75.565) (width 0.25) (layer "F.Cu") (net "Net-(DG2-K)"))
 (segment (start 103.124 82.169) (end 103.124 78.75) (width 0.25) (layer "F.Cu") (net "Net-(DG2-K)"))
 (segment (start 103.642 78.232) (end 103.642 75.565) (width 0.25) (layer "F.Cu") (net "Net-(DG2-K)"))
 (segment (start 103.642 73.035) (end 103.632 73.025) (width 0.25) (layer "F.Cu") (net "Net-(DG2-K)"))
 (segment (start 103.627 73.02) (end 103.632 73.025) (width 0.25) (layer "F.Cu") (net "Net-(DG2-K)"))
 (segment (start 107.823 70.485) (end 106.172 70.485) (width 0.25) (layer "B.Cu") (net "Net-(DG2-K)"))
 (segment (start 103.642 75.956) (end 103.642 75.565) (width 0.25) (layer "B.Cu") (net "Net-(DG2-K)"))
 (segment (start 103.627 67.945) (end 104.852 66.72) (width 0.25) (layer "B.Cu") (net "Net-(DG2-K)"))
 (segment (start 107.823 66.167) (end 107.823 65.405) (width 0.25) (layer "B.Cu") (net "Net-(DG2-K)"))
 (segment (start 107.27 66.72) (end 107.823 66.167) (width 0.25) (layer "B.Cu") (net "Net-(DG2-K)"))
 (segment (start 105.918 78.232) (end 107.823 76.327) (width 0.25) (layer "B.Cu") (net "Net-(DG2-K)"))
 (segment (start 104.852 66.72) (end 107.27 66.72) (width 0.25) (layer "B.Cu") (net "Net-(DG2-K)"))
 (segment (start 107.823 76.327) (end 107.823 75.565) (width 0.25) (layer "B.Cu") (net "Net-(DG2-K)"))
 (segment (start 106.172 70.485) (end 103.632 73.025) (width 0.25) (layer "B.Cu") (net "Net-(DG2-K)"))
 (segment (start 105.918 78.232) (end 103.642 75.956) (width 0.25) (layer "B.Cu") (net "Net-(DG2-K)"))
 (segment (start 103.124 89.789) (end 103.124 92.583) (width 0.25) (layer "F.Cu") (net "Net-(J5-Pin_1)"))
 (segment (start 108.077 82.042) (end 108.204 82.169) (width 0.25) (layer "F.Cu") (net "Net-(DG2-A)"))
 (segment (start 109.438 76.871) (end 109.438 68.87) (width 0.25) (layer "F.Cu") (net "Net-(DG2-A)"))
 (segment (start 109.438 68.87) (end 110.363 67.945) (width 0.25) (layer "F.Cu") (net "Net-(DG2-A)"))
 (segment (start 106.182 76.337) (end 106.182 75.565) (width 0.25) (layer "F.Cu") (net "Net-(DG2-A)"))
 (segment (start 108.077 78.232) (end 109.438 76.871) (width 0.25) (layer "F.Cu") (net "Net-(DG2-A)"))
 (segment (start 108.077 78.232) (end 106.182 76.337) (width 0.25) (layer "F.Cu") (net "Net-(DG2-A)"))
 (segment (start 108.077 78.232) (end 108.077 82.042) (width 0.25) (layer "F.Cu") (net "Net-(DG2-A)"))
 (segment (start 110.363 65.405) (end 110.363 67.945) (width 0.25) (layer "F.Cu") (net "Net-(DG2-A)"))
 (segment (start 105.664 89.789) (end 105.664 92.583) (width 0.25) (layer "F.Cu") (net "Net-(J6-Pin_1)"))
 (segment (start 107.823 67.555) (end 106.167 65.899) (width 0.25) (layer "F.Cu") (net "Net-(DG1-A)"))
 (segment (start 110.744 82.169) (end 110.744 78.613) (width 0.25) (layer "F.Cu") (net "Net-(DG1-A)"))
 (segment (start 110.363 78.232) (end 110.363 75.565) (width 0.25) (layer "F.Cu") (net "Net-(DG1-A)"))
 (segment (start 107.823 67.945) (end 107.823 67.555) (width 0.25) (layer "F.Cu") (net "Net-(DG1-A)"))
 (segment (start 110.363 75.565) (end 110.363 70.485) (width 0.25) (layer "F.Cu") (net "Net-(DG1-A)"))
 (segment (start 110.744 78.613) (end 110.363 78.232) (width 0.25) (layer "F.Cu") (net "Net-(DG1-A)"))
 (segment (start 106.167 65.899) (end 106.167 65.405) (width 0.25) (layer "F.Cu") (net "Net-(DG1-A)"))
 (segment (start 110.363 70.485) (end 107.823 67.945) (width 0.25) (layer "B.Cu") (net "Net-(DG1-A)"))
 (segment (start 110.744 82.169) (end 110.744 80.899) (width 0.25) (layer "B.Cu") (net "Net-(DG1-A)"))
 (segment (start 108.077 78.232) (end 110.363 75.946) (width 0.25) (layer "B.Cu") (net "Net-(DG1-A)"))
 (segment (start 110.363 70.485) (end 107.823 73.025) (width 0.25) (layer "B.Cu") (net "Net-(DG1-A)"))
 (segment (start 107.823 73.025) (end 106.172 73.025) (width 0.25) (layer "B.Cu") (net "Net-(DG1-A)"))
 (segment (start 110.744 80.899) (end 108.077 78.232) (width 0.25) (layer "B.Cu") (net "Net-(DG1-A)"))
 (segment (start 110.363 75.946) (end 110.363 75.565) (width 0.25) (layer "B.Cu") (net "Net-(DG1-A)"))
 (segment (start 104.902 69.21) (end 104.902 77.216) (width 0.25) (layer "F.Cu") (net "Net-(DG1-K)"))
 (segment (start 106.167 67.945) (end 103.627 65.405) (width 0.25) (layer "F.Cu") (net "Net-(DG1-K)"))
 (segment (start 105.664 82.169) (end 105.664 78.486) (width 0.25) (layer "F.Cu") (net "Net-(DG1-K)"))
 (segment (start 104.902 77.216) (end 105.918 78.232) (width 0.25) (layer "F.Cu") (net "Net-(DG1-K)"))
 (segment (start 106.167 67.945) (end 104.902 69.21) (width 0.25) (layer "F.Cu") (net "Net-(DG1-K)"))
 (segment (start 110.744 89.789) (end 110.744 92.583) (width 0.25) (layer "F.Cu") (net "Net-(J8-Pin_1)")))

